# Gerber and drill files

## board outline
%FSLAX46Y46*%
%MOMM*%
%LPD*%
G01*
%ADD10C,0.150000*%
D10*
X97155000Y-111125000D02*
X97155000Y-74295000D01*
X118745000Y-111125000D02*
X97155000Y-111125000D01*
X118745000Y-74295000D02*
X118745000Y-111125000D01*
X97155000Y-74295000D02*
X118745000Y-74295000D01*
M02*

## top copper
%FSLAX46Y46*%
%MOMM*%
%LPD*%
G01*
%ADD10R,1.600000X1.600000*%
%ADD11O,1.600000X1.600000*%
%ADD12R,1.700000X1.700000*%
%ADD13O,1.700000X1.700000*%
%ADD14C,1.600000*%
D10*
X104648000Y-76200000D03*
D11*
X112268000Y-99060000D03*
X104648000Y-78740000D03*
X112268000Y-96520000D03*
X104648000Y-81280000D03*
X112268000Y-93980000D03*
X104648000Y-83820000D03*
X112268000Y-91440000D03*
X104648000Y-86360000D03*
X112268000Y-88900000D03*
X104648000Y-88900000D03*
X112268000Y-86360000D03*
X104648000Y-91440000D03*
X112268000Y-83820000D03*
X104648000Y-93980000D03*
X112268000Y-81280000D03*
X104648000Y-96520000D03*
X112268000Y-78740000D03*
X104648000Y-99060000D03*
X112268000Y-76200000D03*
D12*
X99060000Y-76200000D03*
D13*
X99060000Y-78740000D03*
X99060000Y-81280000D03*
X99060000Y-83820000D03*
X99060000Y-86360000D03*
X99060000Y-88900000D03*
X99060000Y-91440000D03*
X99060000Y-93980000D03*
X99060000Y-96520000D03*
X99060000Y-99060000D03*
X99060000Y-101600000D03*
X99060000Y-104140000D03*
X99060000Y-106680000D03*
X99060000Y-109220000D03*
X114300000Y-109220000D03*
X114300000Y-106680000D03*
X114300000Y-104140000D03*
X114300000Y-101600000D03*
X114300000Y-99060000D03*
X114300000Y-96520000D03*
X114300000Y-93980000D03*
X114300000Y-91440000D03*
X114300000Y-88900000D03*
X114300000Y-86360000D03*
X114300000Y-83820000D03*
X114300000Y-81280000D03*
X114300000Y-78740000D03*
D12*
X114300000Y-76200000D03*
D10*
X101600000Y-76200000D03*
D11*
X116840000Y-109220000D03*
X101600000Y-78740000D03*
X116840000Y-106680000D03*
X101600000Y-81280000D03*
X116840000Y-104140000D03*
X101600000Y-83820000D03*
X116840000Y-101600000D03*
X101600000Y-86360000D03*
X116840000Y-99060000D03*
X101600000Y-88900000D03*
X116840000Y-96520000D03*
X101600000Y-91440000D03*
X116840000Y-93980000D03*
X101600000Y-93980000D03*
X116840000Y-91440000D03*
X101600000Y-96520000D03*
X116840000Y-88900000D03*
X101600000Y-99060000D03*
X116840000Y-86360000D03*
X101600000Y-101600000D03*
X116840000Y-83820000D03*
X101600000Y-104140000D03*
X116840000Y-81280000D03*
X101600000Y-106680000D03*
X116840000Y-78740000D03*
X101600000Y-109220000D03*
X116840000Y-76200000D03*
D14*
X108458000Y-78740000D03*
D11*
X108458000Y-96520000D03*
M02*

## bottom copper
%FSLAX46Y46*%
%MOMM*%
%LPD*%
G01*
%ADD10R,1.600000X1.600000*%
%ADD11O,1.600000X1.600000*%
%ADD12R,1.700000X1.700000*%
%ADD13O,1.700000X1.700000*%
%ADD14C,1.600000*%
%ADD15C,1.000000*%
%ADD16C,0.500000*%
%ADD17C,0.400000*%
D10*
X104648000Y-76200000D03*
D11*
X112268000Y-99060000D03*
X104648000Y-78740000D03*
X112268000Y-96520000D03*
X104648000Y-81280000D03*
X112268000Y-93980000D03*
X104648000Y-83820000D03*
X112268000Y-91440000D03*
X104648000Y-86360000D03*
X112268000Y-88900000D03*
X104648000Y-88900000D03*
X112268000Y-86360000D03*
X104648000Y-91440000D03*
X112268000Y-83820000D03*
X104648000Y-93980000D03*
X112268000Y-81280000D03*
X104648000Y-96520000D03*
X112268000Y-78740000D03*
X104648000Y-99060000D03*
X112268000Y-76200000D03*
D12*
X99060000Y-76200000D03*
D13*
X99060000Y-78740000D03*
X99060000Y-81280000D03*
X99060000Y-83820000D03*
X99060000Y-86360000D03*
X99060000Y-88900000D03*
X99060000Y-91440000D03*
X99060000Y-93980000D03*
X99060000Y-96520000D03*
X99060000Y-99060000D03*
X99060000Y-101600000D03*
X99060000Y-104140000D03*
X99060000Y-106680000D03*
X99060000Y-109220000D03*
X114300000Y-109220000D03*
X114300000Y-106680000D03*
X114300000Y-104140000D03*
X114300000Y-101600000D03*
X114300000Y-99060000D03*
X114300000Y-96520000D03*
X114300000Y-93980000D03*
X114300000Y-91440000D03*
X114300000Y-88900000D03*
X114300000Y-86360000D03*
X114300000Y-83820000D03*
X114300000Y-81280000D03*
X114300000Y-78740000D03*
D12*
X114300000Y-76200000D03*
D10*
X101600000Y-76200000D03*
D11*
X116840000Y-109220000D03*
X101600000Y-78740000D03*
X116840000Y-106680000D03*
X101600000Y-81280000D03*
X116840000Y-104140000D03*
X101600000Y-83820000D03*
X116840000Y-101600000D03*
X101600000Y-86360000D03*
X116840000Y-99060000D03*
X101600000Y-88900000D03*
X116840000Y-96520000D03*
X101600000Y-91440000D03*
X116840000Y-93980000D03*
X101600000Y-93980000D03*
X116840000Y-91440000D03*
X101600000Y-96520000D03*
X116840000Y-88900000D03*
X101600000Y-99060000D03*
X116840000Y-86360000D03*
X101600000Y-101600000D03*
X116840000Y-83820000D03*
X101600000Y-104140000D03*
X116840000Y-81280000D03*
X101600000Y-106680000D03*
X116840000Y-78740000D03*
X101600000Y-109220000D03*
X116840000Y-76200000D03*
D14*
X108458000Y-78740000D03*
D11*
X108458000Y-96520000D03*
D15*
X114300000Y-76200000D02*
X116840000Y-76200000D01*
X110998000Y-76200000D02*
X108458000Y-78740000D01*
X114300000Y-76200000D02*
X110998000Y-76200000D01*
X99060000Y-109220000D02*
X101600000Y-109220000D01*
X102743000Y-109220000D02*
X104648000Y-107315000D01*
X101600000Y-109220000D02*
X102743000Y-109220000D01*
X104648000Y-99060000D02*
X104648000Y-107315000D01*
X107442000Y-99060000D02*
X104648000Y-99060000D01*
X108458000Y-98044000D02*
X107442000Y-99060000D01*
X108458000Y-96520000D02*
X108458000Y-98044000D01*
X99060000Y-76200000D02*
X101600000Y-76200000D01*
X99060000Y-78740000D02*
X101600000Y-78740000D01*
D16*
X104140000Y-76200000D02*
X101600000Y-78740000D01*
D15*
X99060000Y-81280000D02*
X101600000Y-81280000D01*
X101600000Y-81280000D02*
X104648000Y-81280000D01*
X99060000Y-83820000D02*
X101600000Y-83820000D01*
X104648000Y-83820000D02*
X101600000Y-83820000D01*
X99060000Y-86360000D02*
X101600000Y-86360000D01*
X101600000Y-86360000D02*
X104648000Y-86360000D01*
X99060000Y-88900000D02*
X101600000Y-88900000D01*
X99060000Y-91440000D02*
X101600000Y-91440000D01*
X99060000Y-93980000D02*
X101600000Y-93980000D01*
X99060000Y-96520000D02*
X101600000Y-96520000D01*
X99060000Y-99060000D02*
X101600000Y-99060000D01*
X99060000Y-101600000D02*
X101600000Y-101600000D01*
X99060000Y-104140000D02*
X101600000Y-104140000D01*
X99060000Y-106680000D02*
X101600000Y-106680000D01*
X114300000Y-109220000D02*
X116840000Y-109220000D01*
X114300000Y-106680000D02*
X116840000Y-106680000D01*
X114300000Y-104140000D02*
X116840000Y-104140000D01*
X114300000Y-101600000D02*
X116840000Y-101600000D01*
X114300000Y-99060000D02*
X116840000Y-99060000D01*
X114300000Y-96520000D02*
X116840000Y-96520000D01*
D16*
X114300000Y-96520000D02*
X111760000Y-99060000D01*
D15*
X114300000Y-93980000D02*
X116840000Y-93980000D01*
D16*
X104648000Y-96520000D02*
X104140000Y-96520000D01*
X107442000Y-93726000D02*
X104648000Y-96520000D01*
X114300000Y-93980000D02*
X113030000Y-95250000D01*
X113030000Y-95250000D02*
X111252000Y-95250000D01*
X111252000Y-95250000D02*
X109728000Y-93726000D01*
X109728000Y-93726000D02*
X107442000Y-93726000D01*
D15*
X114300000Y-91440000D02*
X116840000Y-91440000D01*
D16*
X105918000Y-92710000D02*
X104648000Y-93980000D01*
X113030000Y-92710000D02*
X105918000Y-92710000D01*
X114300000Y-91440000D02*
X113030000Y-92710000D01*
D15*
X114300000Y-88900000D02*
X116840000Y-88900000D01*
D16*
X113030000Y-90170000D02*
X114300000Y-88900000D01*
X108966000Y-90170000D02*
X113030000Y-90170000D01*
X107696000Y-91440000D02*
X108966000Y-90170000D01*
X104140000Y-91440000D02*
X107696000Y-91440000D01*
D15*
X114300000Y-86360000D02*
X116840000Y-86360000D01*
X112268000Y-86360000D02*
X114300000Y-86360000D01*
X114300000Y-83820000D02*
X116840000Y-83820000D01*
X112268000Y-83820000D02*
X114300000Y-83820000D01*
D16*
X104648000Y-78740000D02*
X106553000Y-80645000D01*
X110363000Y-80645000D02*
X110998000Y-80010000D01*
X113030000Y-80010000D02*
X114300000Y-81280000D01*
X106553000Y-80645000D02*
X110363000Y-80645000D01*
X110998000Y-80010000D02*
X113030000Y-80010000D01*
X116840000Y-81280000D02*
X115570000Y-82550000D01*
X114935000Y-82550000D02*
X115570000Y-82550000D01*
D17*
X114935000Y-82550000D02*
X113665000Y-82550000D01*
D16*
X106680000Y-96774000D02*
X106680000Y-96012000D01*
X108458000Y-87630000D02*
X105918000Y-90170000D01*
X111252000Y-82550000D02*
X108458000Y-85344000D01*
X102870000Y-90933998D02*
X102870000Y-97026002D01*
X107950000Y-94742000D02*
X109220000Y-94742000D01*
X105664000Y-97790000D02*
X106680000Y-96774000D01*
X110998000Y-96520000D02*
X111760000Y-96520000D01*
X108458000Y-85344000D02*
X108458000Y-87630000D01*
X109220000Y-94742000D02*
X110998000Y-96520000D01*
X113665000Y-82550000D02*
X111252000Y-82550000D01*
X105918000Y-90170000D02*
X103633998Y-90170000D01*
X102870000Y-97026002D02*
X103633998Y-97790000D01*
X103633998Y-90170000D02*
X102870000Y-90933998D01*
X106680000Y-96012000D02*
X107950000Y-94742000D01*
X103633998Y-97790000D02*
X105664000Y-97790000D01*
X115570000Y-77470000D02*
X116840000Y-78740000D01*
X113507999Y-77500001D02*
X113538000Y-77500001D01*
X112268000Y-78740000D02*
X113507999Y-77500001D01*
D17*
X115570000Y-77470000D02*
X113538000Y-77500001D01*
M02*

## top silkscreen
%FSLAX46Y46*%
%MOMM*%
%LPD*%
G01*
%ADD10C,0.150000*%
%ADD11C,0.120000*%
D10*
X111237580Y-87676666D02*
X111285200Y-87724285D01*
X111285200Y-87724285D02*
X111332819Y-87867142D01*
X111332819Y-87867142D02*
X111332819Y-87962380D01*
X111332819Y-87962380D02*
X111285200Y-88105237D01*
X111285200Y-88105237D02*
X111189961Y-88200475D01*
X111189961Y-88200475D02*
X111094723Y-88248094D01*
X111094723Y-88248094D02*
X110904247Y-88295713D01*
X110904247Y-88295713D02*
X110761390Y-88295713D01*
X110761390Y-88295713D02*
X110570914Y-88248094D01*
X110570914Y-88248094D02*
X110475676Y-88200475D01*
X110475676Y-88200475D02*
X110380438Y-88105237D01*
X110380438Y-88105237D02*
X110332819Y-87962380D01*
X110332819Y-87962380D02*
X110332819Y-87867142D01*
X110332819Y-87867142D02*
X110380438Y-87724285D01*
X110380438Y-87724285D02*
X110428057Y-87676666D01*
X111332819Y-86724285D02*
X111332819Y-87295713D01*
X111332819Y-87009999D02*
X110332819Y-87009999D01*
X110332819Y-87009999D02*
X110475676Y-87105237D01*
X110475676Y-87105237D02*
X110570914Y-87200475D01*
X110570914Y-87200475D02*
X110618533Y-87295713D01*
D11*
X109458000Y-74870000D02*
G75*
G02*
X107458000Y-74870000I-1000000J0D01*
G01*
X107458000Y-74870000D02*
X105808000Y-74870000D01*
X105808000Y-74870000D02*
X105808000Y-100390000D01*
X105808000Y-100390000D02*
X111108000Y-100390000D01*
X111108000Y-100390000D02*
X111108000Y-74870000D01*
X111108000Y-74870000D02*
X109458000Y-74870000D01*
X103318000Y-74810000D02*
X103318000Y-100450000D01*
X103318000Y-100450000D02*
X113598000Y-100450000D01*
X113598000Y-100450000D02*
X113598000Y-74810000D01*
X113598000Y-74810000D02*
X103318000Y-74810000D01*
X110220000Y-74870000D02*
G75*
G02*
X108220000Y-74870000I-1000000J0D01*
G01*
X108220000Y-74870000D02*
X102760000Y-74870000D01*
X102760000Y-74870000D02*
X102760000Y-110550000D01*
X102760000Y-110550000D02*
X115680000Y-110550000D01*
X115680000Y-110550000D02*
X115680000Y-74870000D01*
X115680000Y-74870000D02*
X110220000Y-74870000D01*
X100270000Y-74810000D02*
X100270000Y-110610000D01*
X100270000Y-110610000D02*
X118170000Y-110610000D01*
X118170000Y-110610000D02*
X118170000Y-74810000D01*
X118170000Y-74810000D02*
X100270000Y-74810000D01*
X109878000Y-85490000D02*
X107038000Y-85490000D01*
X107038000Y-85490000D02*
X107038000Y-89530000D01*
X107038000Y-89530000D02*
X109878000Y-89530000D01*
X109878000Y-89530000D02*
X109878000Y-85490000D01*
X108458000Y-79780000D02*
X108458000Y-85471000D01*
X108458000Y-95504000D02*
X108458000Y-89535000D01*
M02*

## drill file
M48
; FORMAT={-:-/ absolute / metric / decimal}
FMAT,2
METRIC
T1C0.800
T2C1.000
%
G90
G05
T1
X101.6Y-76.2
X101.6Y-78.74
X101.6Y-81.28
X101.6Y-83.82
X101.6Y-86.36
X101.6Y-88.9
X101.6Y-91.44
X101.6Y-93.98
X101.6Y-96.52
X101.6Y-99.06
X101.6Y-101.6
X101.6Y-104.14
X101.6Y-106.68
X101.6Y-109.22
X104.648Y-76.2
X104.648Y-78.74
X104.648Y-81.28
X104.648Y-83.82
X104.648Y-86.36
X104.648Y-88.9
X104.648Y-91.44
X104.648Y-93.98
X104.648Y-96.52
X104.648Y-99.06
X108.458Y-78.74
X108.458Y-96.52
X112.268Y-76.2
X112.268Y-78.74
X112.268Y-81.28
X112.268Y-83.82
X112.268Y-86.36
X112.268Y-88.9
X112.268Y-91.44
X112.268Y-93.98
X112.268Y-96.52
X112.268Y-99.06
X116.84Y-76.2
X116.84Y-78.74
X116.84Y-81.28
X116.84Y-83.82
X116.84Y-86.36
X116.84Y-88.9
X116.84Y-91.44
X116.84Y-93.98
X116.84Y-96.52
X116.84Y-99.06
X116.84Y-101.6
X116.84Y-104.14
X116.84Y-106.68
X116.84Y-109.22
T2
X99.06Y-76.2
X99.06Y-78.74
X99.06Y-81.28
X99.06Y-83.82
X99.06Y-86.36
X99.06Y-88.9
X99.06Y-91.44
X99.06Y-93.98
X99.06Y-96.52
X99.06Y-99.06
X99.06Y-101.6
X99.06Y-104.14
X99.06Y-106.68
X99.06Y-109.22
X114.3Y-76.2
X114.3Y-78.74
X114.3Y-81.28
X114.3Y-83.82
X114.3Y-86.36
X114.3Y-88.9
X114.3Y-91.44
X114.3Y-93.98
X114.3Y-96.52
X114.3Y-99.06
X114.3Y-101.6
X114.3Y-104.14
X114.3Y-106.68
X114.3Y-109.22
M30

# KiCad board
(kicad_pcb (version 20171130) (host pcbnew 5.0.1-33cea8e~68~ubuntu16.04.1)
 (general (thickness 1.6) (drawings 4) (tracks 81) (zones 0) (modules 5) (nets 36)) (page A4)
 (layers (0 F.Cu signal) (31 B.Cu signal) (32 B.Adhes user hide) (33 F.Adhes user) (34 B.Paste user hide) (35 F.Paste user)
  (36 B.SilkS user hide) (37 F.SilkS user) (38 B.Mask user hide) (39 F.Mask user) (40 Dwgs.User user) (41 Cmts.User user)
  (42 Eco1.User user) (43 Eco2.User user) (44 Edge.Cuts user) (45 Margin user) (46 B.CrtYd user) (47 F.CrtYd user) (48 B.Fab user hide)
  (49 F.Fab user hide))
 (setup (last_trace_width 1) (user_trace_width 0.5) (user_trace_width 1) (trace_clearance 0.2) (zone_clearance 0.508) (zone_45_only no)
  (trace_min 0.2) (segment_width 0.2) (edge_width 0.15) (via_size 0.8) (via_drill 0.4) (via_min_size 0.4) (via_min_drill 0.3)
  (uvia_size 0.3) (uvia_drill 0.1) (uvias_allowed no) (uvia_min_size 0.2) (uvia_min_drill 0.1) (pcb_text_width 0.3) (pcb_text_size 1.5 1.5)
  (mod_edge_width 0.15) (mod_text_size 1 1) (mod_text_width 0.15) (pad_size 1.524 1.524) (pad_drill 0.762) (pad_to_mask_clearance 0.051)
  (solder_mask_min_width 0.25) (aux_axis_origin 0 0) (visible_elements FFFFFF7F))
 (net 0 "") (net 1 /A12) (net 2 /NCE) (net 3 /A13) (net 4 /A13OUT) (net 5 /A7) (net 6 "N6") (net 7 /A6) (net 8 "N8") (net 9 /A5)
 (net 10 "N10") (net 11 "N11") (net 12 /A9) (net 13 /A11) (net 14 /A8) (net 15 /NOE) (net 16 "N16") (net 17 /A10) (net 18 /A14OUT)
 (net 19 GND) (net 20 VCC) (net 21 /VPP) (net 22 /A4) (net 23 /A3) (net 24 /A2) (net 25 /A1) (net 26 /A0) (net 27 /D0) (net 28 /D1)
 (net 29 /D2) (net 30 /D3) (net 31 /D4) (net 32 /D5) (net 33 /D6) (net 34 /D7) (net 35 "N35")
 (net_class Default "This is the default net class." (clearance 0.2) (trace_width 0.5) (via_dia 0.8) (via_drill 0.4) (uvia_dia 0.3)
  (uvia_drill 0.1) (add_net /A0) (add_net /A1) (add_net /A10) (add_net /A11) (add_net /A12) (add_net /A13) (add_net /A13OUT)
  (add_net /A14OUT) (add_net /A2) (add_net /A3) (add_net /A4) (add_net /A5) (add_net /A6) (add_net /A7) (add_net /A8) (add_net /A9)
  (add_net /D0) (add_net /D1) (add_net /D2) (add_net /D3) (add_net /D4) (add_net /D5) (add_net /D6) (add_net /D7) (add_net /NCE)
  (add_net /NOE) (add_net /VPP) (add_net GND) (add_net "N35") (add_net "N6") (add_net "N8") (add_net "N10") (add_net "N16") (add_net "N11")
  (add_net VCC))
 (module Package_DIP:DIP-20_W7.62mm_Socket (layer F.Cu) (at 104.648 76.2)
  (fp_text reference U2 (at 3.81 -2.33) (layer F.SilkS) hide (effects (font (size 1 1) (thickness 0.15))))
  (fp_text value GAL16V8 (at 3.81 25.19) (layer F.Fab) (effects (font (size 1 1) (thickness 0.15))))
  (fp_arc (start 3.81 -1.33) (end 2.81 -1.33) (angle -180) (layer F.SilkS) (width 0.12))
  (fp_line (start 2.81 -1.33) (end 1.16 -1.33) (layer F.SilkS) (width 0.12))
  (fp_line (start 1.16 -1.33) (end 1.16 24.19) (layer F.SilkS) (width 0.12))
  (fp_line (start 1.16 24.19) (end 6.46 24.19) (layer F.SilkS) (width 0.12))
  (fp_line (start 6.46 24.19) (end 6.46 -1.33) (layer F.SilkS) (width 0.12))
  (fp_line (start 6.46 -1.33) (end 4.81 -1.33) (layer F.SilkS) (width 0.12))
  (fp_line (start -1.33 -1.39) (end -1.33 24.25) (layer F.SilkS) (width 0.12))
  (fp_line (start -1.33 24.25) (end 8.95 24.25) (layer F.SilkS) (width 0.12))
  (fp_line (start 8.95 24.25) (end 8.95 -1.39) (layer F.SilkS) (width 0.12))
  (fp_line (start 8.95 -1.39) (end -1.33 -1.39) (layer F.SilkS) (width 0.12))
  (pad 1 thru_hole rect (at 0 0) (size 1.6 1.6) (drill 0.8) (layers *.Cu *.Mask) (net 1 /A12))
  (pad 11 thru_hole oval (at 7.62 22.86) (size 1.6 1.6) (drill 0.8) (layers *.Cu *.Mask) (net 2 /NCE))
  (pad 2 thru_hole oval (at 0 2.54) (size 1.6 1.6) (drill 0.8) (layers *.Cu *.Mask) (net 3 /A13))
  (pad 12 thru_hole oval (at 7.62 20.32) (size 1.6 1.6) (drill 0.8) (layers *.Cu *.Mask) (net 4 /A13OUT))
  (pad 3 thru_hole oval (at 0 5.08) (size 1.6 1.6) (drill 0.8) (layers *.Cu *.Mask) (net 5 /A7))
  (pad 13 thru_hole oval (at 7.62 17.78) (size 1.6 1.6) (drill 0.8) (layers *.Cu *.Mask) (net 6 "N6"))
  (pad 4 thru_hole oval (at 0 7.62) (size 1.6 1.6) (drill 0.8) (layers *.Cu *.Mask) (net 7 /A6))
  (pad 14 thru_hole oval (at 7.62 15.24) (size 1.6 1.6) (drill 0.8) (layers *.Cu *.Mask) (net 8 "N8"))
  (pad 5 thru_hole oval (at 0 10.16) (size 1.6 1.6) (drill 0.8) (layers *.Cu *.Mask) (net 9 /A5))
  (pad 15 thru_hole oval (at 7.62 12.7) (size 1.6 1.6) (drill 0.8) (layers *.Cu *.Mask) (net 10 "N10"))
  (pad 6 thru_hole oval (at 0 12.7) (size 1.6 1.6) (drill 0.8) (layers *.Cu *.Mask) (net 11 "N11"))
  (pad 16 thru_hole oval (at 7.62 10.16) (size 1.6 1.6) (drill 0.8) (layers *.Cu *.Mask) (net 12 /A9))
  (pad 7 thru_hole oval (at 0 15.24) (size 1.6 1.6) (drill 0.8) (layers *.Cu *.Mask) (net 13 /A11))
  (pad 17 thru_hole oval (at 7.62 7.62) (size 1.6 1.6) (drill 0.8) (layers *.Cu *.Mask) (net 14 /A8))
  (pad 8 thru_hole oval (at 0 17.78) (size 1.6 1.6) (drill 0.8) (layers *.Cu *.Mask) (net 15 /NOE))
  (pad 18 thru_hole oval (at 7.62 5.08) (size 1.6 1.6) (drill 0.8) (layers *.Cu *.Mask) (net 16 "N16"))
  (pad 9 thru_hole oval (at 0 20.32) (size 1.6 1.6) (drill 0.8) (layers *.Cu *.Mask) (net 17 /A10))
  (pad 19 thru_hole oval (at 7.62 2.54) (size 1.6 1.6) (drill 0.8) (layers *.Cu *.Mask) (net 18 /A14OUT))
  (pad 10 thru_hole oval (at 0 22.86) (size 1.6 1.6) (drill 0.8) (layers *.Cu *.Mask) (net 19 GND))
  (pad 20 thru_hole oval (at 7.62 0) (size 1.6 1.6) (drill 0.8) (layers *.Cu *.Mask) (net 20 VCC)))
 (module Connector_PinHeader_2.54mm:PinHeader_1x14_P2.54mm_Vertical (layer B.Cu) (at 99.06 76.2 180)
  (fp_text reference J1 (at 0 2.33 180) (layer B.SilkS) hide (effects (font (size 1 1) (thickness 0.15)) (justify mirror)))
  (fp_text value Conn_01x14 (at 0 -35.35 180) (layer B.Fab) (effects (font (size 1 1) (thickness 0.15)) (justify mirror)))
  (pad 1 thru_hole rect (at 0 0 180) (size 1.7 1.7) (drill 1) (layers *.Cu *.Mask) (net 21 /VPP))
  (pad 2 thru_hole oval (at 0 -2.54 180) (size 1.7 1.7) (drill 1) (layers *.Cu *.Mask) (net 1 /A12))
  (pad 3 thru_hole oval (at 0 -5.08 180) (size 1.7 1.7) (drill 1) (layers *.Cu *.Mask) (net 5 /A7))
  (pad 4 thru_hole oval (at 0 -7.62 180) (size 1.7 1.7) (drill 1) (layers *.Cu *.Mask) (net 7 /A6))
  (pad 5 thru_hole oval (at 0 -10.16 180) (size 1.7 1.7) (drill 1) (layers *.Cu *.Mask) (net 9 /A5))
  (pad 6 thru_hole oval (at 0 -12.7 180) (size 1.7 1.7) (drill 1) (layers *.Cu *.Mask) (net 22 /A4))
  (pad 7 thru_hole oval (at 0 -15.24 180) (size 1.7 1.7) (drill 1) (layers *.Cu *.Mask) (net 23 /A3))
  (pad 8 thru_hole oval (at 0 -17.78 180) (size 1.7 1.7) (drill 1) (layers *.Cu *.Mask) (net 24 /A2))
  (pad 9 thru_hole oval (at 0 -20.32 180) (size 1.7 1.7) (drill 1) (layers *.Cu *.Mask) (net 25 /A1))
  (pad 10 thru_hole oval (at 0 -22.86 180) (size 1.7 1.7) (drill 1) (layers *.Cu *.Mask) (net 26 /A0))
  (pad 11 thru_hole oval (at 0 -25.4 180) (size 1.7 1.7) (drill 1) (layers *.Cu *.Mask) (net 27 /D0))
  (pad 12 thru_hole oval (at 0 -27.94 180) (size 1.7 1.7) (drill 1) (layers *.Cu *.Mask) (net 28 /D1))
  (pad 13 thru_hole oval (at 0 -30.48 180) (size 1.7 1.7) (drill 1) (layers *.Cu *.Mask) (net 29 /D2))
  (pad 14 thru_hole oval (at 0 -33.02 180) (size 1.7 1.7) (drill 1) (layers *.Cu *.Mask) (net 19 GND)))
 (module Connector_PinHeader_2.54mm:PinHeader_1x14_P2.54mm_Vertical (layer B.Cu) (at 114.3 76.2 180)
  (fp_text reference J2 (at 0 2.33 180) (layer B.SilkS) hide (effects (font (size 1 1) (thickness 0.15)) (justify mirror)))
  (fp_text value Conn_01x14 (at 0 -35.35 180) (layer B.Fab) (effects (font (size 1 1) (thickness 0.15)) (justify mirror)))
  (pad 14 thru_hole oval (at 0 -33.02 180) (size 1.7 1.7) (drill 1) (layers *.Cu *.Mask) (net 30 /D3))
  (pad 13 thru_hole oval (at 0 -30.48 180) (size 1.7 1.7) (drill 1) (layers *.Cu *.Mask) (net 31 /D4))
  (pad 12 thru_hole oval (at 0 -27.94 180) (size 1.7 1.7) (drill 1) (layers *.Cu *.Mask) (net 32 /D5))
  (pad 11 thru_hole oval (at 0 -25.4 180) (size 1.7 1.7) (drill 1) (layers *.Cu *.Mask) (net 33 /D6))
  (pad 10 thru_hole oval (at 0 -22.86 180) (size 1.7 1.7) (drill 1) (layers *.Cu *.Mask) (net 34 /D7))
  (pad 9 thru_hole oval (at 0 -20.32 180) (size 1.7 1.7) (drill 1) (layers *.Cu *.Mask) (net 2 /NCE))
  (pad 8 thru_hole oval (at 0 -17.78 180) (size 1.7 1.7) (drill 1) (layers *.Cu *.Mask) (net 17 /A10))
  (pad 7 thru_hole oval (at 0 -15.24 180) (size 1.7 1.7) (drill 1) (layers *.Cu *.Mask) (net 15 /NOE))
  (pad 6 thru_hole oval (at 0 -12.7 180) (size 1.7 1.7) (drill 1) (layers *.Cu *.Mask) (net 13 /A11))
  (pad 5 thru_hole oval (at 0 -10.16 180) (size 1.7 1.7) (drill 1) (layers *.Cu *.Mask) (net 12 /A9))
  (pad 4 thru_hole oval (at 0 -7.62 180) (size 1.7 1.7) (drill 1) (layers *.Cu *.Mask) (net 14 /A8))
  (pad 3 thru_hole oval (at 0 -5.08 180) (size 1.7 1.7) (drill 1) (layers *.Cu *.Mask) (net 3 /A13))
  (pad 2 thru_hole oval (at 0 -2.54 180) (size 1.7 1.7) (drill 1) (layers *.Cu *.Mask) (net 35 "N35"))
  (pad 1 thru_hole rect (at 0 0 180) (size 1.7 1.7) (drill 1) (layers *.Cu *.Mask) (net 20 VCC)))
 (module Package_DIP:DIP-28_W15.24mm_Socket (layer F.Cu) (at 101.6 76.2)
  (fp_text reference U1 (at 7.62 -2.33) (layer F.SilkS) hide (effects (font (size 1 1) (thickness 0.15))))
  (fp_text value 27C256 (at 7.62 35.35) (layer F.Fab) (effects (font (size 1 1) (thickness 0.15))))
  (fp_arc (start 7.62 -1.33) (end 6.62 -1.33) (angle -180) (layer F.SilkS) (width 0.12))
  (fp_line (start 6.62 -1.33) (end 1.16 -1.33) (layer F.SilkS) (width 0.12))
  (fp_line (start 1.16 -1.33) (end 1.16 34.35) (layer F.SilkS) (width 0.12))
  (fp_line (start 1.16 34.35) (end 14.08 34.35) (layer F.SilkS) (width 0.12))
  (fp_line (start 14.08 34.35) (end 14.08 -1.33) (layer F.SilkS) (width 0.12))
  (fp_line (start 14.08 -1.33) (end 8.62 -1.33) (layer F.SilkS) (width 0.12))
  (fp_line (start -1.33 -1.39) (end -1.33 34.41) (layer F.SilkS) (width 0.12))
  (fp_line (start -1.33 34.41) (end 16.57 34.41) (layer F.SilkS) (width 0.12))
  (fp_line (start 16.57 34.41) (end 16.57 -1.39) (layer F.SilkS) (width 0.12))
  (fp_line (start 16.57 -1.39) (end -1.33 -1.39) (layer F.SilkS) (width 0.12))
  (pad 1 thru_hole rect (at 0 0) (size 1.6 1.6) (drill 0.8) (layers *.Cu *.Mask) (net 21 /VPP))
  (pad 15 thru_hole oval (at 15.24 33.02) (size 1.6 1.6) (drill 0.8) (layers *.Cu *.Mask) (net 30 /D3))
  (pad 2 thru_hole oval (at 0 2.54) (size 1.6 1.6) (drill 0.8) (layers *.Cu *.Mask) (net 1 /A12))
  (pad 16 thru_hole oval (at 15.24 30.48) (size 1.6 1.6) (drill 0.8) (layers *.Cu *.Mask) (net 31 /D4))
  (pad 3 thru_hole oval (at 0 5.08) (size 1.6 1.6) (drill 0.8) (layers *.Cu *.Mask) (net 5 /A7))
  (pad 17 thru_hole oval (at 15.24 27.94) (size 1.6 1.6) (drill 0.8) (layers *.Cu *.Mask) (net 32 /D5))
  (pad 4 thru_hole oval (at 0 7.62) (size 1.6 1.6) (drill 0.8) (layers *.Cu *.Mask) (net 7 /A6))
  (pad 18 thru_hole oval (at 15.24 25.4) (size 1.6 1.6) (drill 0.8) (layers *.Cu *.Mask) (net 33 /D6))
  (pad 5 thru_hole oval (at 0 10.16) (size 1.6 1.6) (drill 0.8) (layers *.Cu *.Mask) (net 9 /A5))
  (pad 19 thru_hole oval (at 15.24 22.86) (size 1.6 1.6) (drill 0.8) (layers *.Cu *.Mask) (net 34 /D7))
  (pad 6 thru_hole oval (at 0 12.7) (size 1.6 1.6) (drill 0.8) (layers *.Cu *.Mask) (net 22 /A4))
  (pad 20 thru_hole oval (at 15.24 20.32) (size 1.6 1.6) (drill 0.8) (layers *.Cu *.Mask) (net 2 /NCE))
  (pad 7 thru_hole oval (at 0 15.24) (size 1.6 1.6) (drill 0.8) (layers *.Cu *.Mask) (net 23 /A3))
  (pad 21 thru_hole oval (at 15.24 17.78) (size 1.6 1.6) (drill 0.8) (layers *.Cu *.Mask) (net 17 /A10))
  (pad 8 thru_hole oval (at 0 17.78) (size 1.6 1.6) (drill 0.8) (layers *.Cu *.Mask) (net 24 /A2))
  (pad 22 thru_hole oval (at 15.24 15.24) (size 1.6 1.6) (drill 0.8) (layers *.Cu *.Mask) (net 15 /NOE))
  (pad 9 thru_hole oval (at 0 20.32) (size 1.6 1.6) (drill 0.8) (layers *.Cu *.Mask) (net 25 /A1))
  (pad 23 thru_hole oval (at 15.24 12.7) (size 1.6 1.6) (drill 0.8) (layers *.Cu *.Mask) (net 13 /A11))
  (pad 10 thru_hole oval (at 0 22.86) (size 1.6 1.6) (drill 0.8) (layers *.Cu *.Mask) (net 26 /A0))
  (pad 24 thru_hole oval (at 15.24 10.16) (size 1.6 1.6) (drill 0.8) (layers *.Cu *.Mask) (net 12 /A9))
  (pad 11 thru_hole oval (at 0 25.4) (size 1.6 1.6) (drill 0.8) (layers *.Cu *.Mask) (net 27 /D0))
  (pad 25 thru_hole oval (at 15.24 7.62) (size 1.6 1.6) (drill 0.8) (layers *.Cu *.Mask) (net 14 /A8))
  (pad 12 thru_hole oval (at 0 27.94) (size 1.6 1.6) (drill 0.8) (layers *.Cu *.Mask) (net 28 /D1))
  (pad 26 thru_hole oval (at 15.24 5.08) (size 1.6 1.6) (drill 0.8) (layers *.Cu *.Mask) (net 4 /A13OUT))
  (pad 13 thru_hole oval (at 0 30.48) (size 1.6 1.6) (drill 0.8) (layers *.Cu *.Mask) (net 29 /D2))
  (pad 27 thru_hole oval (at 15.24 2.54) (size 1.6 1.6) (drill 0.8) (layers *.Cu *.Mask) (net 18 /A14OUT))
  (pad 14 thru_hole oval (at 0 33.02) (size 1.6 1.6) (drill 0.8) (layers *.Cu *.Mask) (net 19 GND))
  (pad 28 thru_hole oval (at 15.24 0) (size 1.6 1.6) (drill 0.8) (layers *.Cu *.Mask) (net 20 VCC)))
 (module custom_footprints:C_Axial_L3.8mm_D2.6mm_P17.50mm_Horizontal (layer F.Cu) (at 108.458 78.74 270)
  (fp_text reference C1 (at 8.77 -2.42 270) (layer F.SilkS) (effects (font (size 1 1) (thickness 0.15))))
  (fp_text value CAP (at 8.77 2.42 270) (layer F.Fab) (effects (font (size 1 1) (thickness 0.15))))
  (fp_line (start 6.75 -1.42) (end 6.75 1.42) (layer F.SilkS) (width 0.12))
  (fp_line (start 6.75 1.42) (end 10.79 1.42) (layer F.SilkS) (width 0.12))
  (fp_line (start 10.79 1.42) (end 10.79 -1.42) (layer F.SilkS) (width 0.12))
  (fp_line (start 10.79 -1.42) (end 6.75 -1.42) (layer F.SilkS) (width 0.12))
  (fp_line (start 1.04 0) (end 6.731 0) (layer F.SilkS) (width 0.12))
  (fp_line (start 16.764 0) (end 10.795 0) (layer F.SilkS) (width 0.12))
  (pad 1 thru_hole circle (at 0 0 270) (size 1.6 1.6) (drill 0.8) (layers *.Cu *.Mask) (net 20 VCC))
  (pad 2 thru_hole oval (at 17.78 0 270) (size 1.6 1.6) (drill 0.8) (layers *.Cu *.Mask) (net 19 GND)))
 (gr_line (start 97.155 111.125) (end 97.155 74.295) (layer Edge.Cuts) (width 0.15))
 (gr_line (start 118.745 111.125) (end 97.155 111.125) (layer Edge.Cuts) (width 0.15))
 (gr_line (start 118.745 74.295) (end 118.745 111.125) (layer Edge.Cuts) (width 0.15))
 (gr_line (start 97.155 74.295) (end 118.745 74.295) (layer Edge.Cuts) (width 0.15))
 (segment (start 114.3 76.2) (end 116.84 76.2) (width 1) (layer B.Cu) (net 20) (status 30))
 (segment (start 110.998 76.2) (end 108.458 78.74) (width 1) (layer B.Cu) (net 20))
 (segment (start 114.3 76.2) (end 110.998 76.2) (width 1) (layer B.Cu) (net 20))
 (segment (start 99.06 109.22) (end 101.6 109.22) (width 1) (layer B.Cu) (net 19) (status 30))
 (segment (start 102.743 109.22) (end 104.648 107.315) (width 1) (layer B.Cu) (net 19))
 (segment (start 101.6 109.22) (end 102.743 109.22) (width 1) (layer B.Cu) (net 19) (status 10))
 (segment (start 104.648 99.06) (end 104.648 107.315) (width 1) (layer B.Cu) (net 19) (status 10))
 (segment (start 107.442 99.06) (end 104.648 99.06) (width 1) (layer B.Cu) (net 19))
 (segment (start 108.458 98.044) (end 107.442 99.06) (width 1) (layer B.Cu) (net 19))
 (segment (start 108.458 96.52) (end 108.458 98.044) (width 1) (layer B.Cu) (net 19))
 (segment (start 99.06 76.2) (end 101.6 76.2) (width 1) (layer B.Cu) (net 21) (status 30))
 (segment (start 99.06 78.74) (end 101.6 78.74) (width 1) (layer B.Cu) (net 1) (status 30))
 (segment (start 104.14 76.2) (end 101.6 78.74) (width 0.5) (layer B.Cu) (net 1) (status 30))
 (segment (start 99.06 81.28) (end 101.6 81.28) (width 1) (layer B.Cu) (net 5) (status 30))
 (segment (start 101.6 81.28) (end 104.648 81.28) (width 1) (layer B.Cu) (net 5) (status 30))
 (segment (start 99.06 83.82) (end 101.6 83.82) (width 1) (layer B.Cu) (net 7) (status 30))
 (segment (start 104.648 83.82) (end 101.6 83.82) (width 1) (layer B.Cu) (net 7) (status 30))
 (segment (start 99.06 86.36) (end 101.6 86.36) (width 1) (layer B.Cu) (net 9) (status 30))
 (segment (start 101.6 86.36) (end 104.648 86.36) (width 1) (layer B.Cu) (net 9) (status 30))
 (segment (start 99.06 88.9) (end 101.6 88.9) (width 1) (layer B.Cu) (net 22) (status 30))
 (segment (start 99.06 91.44) (end 101.6 91.44) (width 1) (layer B.Cu) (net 23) (status 30))
 (segment (start 99.06 93.98) (end 101.6 93.98) (width 1) (layer B.Cu) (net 24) (status 30))
 (segment (start 99.06 96.52) (end 101.6 96.52) (width 1) (layer B.Cu) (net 25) (status 30))
 (segment (start 99.06 99.06) (end 101.6 99.06) (width 1) (layer B.Cu) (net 26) (status 30))
 (segment (start 99.06 101.6) (end 101.6 101.6) (width 1) (layer B.Cu) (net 27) (status 30))
 (segment (start 99.06 104.14) (end 101.6 104.14) (width 1) (layer B.Cu) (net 28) (status 30))
 (segment (start 99.06 106.68) (end 101.6 106.68) (width 1) (layer B.Cu) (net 29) (status 30))
 (segment (start 114.3 109.22) (end 116.84 109.22) (width 1) (layer B.Cu) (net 30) (status 30))
 (segment (start 114.3 106.68) (end 116.84 106.68) (width 1) (layer B.Cu) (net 31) (status 30))
 (segment (start 114.3 104.14) (end 116.84 104.14) (width 1) (layer B.Cu) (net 32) (status 30))
 (segment (start 114.3 101.6) (end 116.84 101.6) (width 1) (layer B.Cu) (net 33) (status 30))
 (segment (start 114.3 99.06) (end 116.84 99.06) (width 1) (layer B.Cu) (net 34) (status 30))
 (segment (start 114.3 96.52) (end 116.84 96.52) (width 1) (layer B.Cu) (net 2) (status 30))
 (segment (start 114.3 96.52) (end 111.76 99.06) (width 0.5) (layer B.Cu) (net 2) (status 30))
 (segment (start 114.3 93.98) (end 116.84 93.98) (width 1) (layer B.Cu) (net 17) (status 30))
 (segment (start 104.648 96.52) (end 104.14 96.52) (width 0.5) (layer B.Cu) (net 17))
 (segment (start 107.442 93.726) (end 104.648 96.52) (width 0.5) (layer B.Cu) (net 17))
 (segment (start 114.3 93.98) (end 113.03 95.25) (width 0.5) (layer B.Cu) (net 17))
 (segment (start 113.03 95.25) (end 111.252 95.25) (width 0.5) (layer B.Cu) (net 17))
 (segment (start 111.252 95.25) (end 109.728 93.726) (width 0.5) (layer B.Cu) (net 17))
 (segment (start 109.728 93.726) (end 107.442 93.726) (width 0.5) (layer B.Cu) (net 17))
 (segment (start 114.3 91.44) (end 116.84 91.44) (width 1) (layer B.Cu) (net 15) (status 30))
 (segment (start 105.918 92.71) (end 104.648 93.98) (width 0.5) (layer B.Cu) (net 15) (status 20))
 (segment (start 113.03 92.71) (end 105.918 92.71) (width 0.5) (layer B.Cu) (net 15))
 (segment (start 114.3 91.44) (end 113.03 92.71) (width 0.5) (layer B.Cu) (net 15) (status 10))
 (segment (start 114.3 88.9) (end 116.84 88.9) (width 1) (layer B.Cu) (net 13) (status 30))
 (segment (start 113.03 90.17) (end 114.3 88.9) (width 0.5) (layer B.Cu) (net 13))
 (segment (start 108.966 90.17) (end 113.03 90.17) (width 0.5) (layer B.Cu) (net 13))
 (segment (start 107.696 91.44) (end 108.966 90.17) (width 0.5) (layer B.Cu) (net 13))
 (segment (start 104.14 91.44) (end 107.696 91.44) (width 0.5) (layer B.Cu) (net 13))
 (segment (start 114.3 86.36) (end 116.84 86.36) (width 1) (layer B.Cu) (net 12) (status 30))
 (segment (start 112.268 86.36) (end 114.3 86.36) (width 1) (layer B.Cu) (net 12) (status 30))
 (segment (start 114.3 83.82) (end 116.84 83.82) (width 1) (layer B.Cu) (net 14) (status 30))
 (segment (start 112.268 83.82) (end 114.3 83.82) (width 1) (layer B.Cu) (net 14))
 (segment (start 104.648 78.74) (end 106.553 80.645) (width 0.5) (layer B.Cu) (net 3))
 (segment (start 110.363 80.645) (end 110.998 80.01) (width 0.5) (layer B.Cu) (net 3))
 (segment (start 113.03 80.01) (end 114.3 81.28) (width 0.5) (layer B.Cu) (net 3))
 (segment (start 106.553 80.645) (end 110.363 80.645) (width 0.5) (layer B.Cu) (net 3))
 (segment (start 110.998 80.01) (end 113.03 80.01) (width 0.5) (layer B.Cu) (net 3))
 (segment (start 116.84 81.28) (end 115.57 82.55) (width 0.5) (layer B.Cu) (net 4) (status 10))
 (segment (start 114.935 82.55) (end 115.57 82.55) (width 0.5) (layer B.Cu) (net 4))
 (segment (start 114.935 82.55) (end 113.665 82.55) (width 0.4) (layer B.Cu) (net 4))
 (segment (start 106.68 96.774) (end 106.68 96.012) (width 0.5) (layer B.Cu) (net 4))
 (segment (start 108.458 87.63) (end 105.918 90.17) (width 0.5) (layer B.Cu) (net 4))
 (segment (start 111.252 82.55) (end 108.458 85.344) (width 0.5) (layer B.Cu) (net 4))
 (segment (start 102.87 90.933998) (end 102.87 97.026002) (width 0.5) (layer B.Cu) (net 4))
 (segment (start 107.95 94.742) (end 109.22 94.742) (width 0.5) (layer B.Cu) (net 4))
 (segment (start 105.664 97.79) (end 106.68 96.774) (width 0.5) (layer B.Cu) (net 4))
 (segment (start 110.998 96.52) (end 111.76 96.52) (width 0.5) (layer B.Cu) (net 4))
 (segment (start 108.458 85.344) (end 108.458 87.63) (width 0.5) (layer B.Cu) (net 4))
 (segment (start 109.22 94.742) (end 110.998 96.52) (width 0.5) (layer B.Cu) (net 4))
 (segment (start 113.665 82.55) (end 111.252 82.55) (width 0.5) (layer B.Cu) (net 4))
 (segment (start 105.918 90.17) (end 103.633998 90.17) (width 0.5) (layer B.Cu) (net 4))
 (segment (start 102.87 97.026002) (end 103.633998 97.79) (width 0.5) (layer B.Cu) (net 4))
 (segment (start 103.633998 90.17) (end 102.87 90.933998) (width 0.5) (layer B.Cu) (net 4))
 (segment (start 106.68 96.012) (end 107.95 94.742) (width 0.5) (layer B.Cu) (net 4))
 (segment (start 103.633998 97.79) (end 105.664 97.79) (width 0.5) (layer B.Cu) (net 4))
 (segment (start 115.57 77.47) (end 116.84 78.74) (width 0.5) (layer B.Cu) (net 18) (status 20))
 (segment (start 113.507999 77.500001) (end 113.538 77.500001) (width 0.5) (layer B.Cu) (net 18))
 (segment (start 112.268 78.74) (end 113.507999 77.500001) (width 0.5) (layer B.Cu) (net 18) (status 10))
 (segment (start 115.57 77.47) (end 113.538 77.500001) (width 0.4) (layer B.Cu) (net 18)))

